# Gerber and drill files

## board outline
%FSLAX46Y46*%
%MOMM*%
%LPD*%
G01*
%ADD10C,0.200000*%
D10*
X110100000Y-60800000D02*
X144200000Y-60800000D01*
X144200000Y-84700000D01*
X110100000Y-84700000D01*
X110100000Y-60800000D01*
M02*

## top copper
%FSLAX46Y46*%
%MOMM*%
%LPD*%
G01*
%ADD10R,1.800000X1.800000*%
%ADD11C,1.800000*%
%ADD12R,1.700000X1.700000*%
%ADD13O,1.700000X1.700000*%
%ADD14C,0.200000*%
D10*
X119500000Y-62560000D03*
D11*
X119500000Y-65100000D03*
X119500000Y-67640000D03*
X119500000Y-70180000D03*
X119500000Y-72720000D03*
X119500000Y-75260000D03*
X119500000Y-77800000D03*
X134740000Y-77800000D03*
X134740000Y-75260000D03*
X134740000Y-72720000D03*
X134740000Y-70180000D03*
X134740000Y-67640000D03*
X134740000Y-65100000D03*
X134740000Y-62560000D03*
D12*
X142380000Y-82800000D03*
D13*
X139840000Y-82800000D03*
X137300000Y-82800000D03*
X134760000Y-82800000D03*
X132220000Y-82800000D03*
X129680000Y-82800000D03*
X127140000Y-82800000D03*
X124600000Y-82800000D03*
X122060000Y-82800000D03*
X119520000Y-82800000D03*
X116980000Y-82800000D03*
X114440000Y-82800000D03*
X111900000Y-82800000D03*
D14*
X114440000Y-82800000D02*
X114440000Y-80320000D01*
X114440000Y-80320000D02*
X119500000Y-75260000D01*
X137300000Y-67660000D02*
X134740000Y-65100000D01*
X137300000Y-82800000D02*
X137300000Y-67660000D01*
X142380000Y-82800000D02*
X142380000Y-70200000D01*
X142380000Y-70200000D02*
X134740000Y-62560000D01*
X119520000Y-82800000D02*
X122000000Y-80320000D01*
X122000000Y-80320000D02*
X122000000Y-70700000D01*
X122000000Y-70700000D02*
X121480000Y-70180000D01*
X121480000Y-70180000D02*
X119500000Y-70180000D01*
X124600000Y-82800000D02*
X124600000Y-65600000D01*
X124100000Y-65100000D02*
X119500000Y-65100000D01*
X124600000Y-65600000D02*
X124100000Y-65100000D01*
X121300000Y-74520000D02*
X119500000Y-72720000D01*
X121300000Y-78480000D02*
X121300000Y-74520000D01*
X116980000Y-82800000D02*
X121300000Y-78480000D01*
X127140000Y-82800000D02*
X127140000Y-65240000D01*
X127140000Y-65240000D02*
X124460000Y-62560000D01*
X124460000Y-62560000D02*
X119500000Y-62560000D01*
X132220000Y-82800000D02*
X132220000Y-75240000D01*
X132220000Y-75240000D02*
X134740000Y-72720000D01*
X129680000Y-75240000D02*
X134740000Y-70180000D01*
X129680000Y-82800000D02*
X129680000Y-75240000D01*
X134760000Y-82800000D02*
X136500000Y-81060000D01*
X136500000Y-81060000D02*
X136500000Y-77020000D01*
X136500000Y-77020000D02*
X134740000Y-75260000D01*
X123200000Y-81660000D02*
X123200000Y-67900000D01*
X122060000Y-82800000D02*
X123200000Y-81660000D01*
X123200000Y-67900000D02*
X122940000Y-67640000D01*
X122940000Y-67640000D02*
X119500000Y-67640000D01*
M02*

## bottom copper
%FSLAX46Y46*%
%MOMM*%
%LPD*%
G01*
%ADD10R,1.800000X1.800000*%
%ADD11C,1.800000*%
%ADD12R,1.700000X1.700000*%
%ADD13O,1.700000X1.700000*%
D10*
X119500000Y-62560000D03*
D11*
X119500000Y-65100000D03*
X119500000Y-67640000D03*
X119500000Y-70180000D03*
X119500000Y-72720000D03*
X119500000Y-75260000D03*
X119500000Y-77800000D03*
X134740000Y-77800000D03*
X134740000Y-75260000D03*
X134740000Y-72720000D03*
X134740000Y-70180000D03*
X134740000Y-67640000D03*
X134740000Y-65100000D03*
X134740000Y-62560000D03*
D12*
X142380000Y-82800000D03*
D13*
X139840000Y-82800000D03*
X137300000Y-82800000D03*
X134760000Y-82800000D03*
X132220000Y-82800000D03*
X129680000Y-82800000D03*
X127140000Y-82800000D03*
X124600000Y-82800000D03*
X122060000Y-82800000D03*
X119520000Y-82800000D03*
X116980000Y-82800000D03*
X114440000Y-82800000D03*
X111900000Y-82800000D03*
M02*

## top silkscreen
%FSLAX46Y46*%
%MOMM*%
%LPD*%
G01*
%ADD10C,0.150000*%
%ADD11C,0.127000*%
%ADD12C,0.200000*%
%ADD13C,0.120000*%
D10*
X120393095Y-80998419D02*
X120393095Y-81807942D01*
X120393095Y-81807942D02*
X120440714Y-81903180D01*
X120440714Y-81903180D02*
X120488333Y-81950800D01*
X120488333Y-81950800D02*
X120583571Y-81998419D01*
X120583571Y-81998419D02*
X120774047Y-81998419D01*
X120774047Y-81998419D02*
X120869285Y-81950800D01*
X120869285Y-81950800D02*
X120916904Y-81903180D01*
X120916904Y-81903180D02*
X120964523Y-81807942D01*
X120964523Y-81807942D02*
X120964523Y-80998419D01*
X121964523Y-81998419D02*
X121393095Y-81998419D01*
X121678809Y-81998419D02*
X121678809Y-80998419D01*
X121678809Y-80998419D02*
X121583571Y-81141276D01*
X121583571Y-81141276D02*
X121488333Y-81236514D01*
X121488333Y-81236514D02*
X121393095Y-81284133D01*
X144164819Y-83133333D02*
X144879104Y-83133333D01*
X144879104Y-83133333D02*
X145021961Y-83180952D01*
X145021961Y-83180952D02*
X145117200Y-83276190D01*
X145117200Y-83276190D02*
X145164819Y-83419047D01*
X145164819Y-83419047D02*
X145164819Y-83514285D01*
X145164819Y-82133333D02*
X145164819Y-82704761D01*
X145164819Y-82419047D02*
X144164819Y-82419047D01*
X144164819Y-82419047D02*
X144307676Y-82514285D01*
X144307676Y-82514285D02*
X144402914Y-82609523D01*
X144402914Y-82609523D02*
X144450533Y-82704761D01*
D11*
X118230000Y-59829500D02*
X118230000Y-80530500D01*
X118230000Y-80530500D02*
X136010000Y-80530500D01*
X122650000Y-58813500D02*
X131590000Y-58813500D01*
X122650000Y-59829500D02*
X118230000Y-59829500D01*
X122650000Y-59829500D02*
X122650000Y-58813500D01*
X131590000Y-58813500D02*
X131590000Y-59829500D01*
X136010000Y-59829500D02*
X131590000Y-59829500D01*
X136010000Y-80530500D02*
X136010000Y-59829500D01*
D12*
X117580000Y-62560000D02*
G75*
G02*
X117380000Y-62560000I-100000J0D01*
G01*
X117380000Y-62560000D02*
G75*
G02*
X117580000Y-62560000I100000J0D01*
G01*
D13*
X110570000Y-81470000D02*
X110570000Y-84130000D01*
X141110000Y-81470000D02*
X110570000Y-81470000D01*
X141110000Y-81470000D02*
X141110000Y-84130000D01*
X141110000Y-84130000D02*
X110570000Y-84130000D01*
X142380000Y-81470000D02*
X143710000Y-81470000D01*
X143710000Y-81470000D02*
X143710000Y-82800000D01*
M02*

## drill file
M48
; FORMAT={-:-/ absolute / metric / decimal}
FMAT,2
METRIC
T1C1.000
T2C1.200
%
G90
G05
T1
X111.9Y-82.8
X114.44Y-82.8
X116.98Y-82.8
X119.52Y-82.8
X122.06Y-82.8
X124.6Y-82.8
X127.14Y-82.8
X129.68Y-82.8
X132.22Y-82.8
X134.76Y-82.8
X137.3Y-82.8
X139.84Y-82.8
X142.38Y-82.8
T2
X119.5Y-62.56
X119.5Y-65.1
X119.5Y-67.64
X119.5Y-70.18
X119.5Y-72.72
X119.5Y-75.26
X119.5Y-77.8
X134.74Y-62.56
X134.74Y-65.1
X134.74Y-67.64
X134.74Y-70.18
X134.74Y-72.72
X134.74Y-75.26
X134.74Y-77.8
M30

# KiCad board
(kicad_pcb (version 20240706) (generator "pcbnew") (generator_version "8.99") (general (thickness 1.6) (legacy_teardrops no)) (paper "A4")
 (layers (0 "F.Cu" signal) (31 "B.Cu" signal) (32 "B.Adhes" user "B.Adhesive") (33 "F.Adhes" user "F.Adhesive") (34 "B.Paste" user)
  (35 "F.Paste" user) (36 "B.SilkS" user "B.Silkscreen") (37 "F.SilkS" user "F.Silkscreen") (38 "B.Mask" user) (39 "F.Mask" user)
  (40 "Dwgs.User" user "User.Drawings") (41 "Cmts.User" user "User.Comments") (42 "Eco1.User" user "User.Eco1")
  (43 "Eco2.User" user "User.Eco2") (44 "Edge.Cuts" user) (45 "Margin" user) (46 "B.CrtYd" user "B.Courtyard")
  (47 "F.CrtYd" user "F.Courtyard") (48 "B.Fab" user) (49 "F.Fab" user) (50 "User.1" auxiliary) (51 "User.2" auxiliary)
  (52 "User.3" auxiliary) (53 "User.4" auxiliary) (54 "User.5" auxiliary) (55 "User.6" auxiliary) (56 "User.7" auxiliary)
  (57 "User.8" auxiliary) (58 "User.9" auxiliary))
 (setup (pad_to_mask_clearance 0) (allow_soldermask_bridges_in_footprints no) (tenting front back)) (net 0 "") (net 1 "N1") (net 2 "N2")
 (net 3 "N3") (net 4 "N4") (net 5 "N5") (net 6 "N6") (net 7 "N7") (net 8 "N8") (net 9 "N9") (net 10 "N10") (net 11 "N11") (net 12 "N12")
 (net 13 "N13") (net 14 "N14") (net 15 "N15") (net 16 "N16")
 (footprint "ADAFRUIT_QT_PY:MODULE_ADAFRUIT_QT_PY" (layer "F.Cu") (at 127.12 70.18)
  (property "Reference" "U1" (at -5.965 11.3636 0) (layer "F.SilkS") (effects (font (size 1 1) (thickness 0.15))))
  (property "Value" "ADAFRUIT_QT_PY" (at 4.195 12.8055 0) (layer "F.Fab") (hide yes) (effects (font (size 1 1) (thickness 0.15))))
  (fp_line (start -8.89 -10.3505) (end -8.89 10.3505) (stroke (width 0.127) (type solid)) (layer "F.SilkS"))
  (fp_line (start -8.89 10.3505) (end 8.89 10.3505) (stroke (width 0.127) (type solid)) (layer "F.SilkS"))
  (fp_line (start -4.47 -11.3665) (end 4.47 -11.3665) (stroke (width 0.127) (type solid)) (layer "F.SilkS"))
  (fp_line (start -4.47 -10.3505) (end -8.89 -10.3505) (stroke (width 0.127) (type solid)) (layer "F.SilkS"))
  (fp_line (start -4.47 -10.3505) (end -4.47 -11.3665) (stroke (width 0.127) (type solid)) (layer "F.SilkS"))
  (fp_line (start 4.47 -11.3665) (end 4.47 -10.3505) (stroke (width 0.127) (type solid)) (layer "F.SilkS"))
  (fp_line (start 8.89 -10.3505) (end 4.47 -10.3505) (stroke (width 0.127) (type solid)) (layer "F.SilkS"))
  (fp_line (start 8.89 10.3505) (end 8.89 -10.3505) (stroke (width 0.127) (type solid)) (layer "F.SilkS"))
  (fp_circle (center -9.64 -7.62) (end -9.54 -7.62) (stroke (width 0.2) (type solid)) (fill none) (layer "F.SilkS"))
  (pad "1" thru_hole rect (at -7.62 -7.62) (size 1.8 1.8) (drill 1.2) (layers "*.Cu" "*.Mask") (remove_unused_layers no) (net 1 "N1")
   (solder_mask_margin 0.102))
  (pad "2" thru_hole circle (at -7.62 -5.08) (size 1.8 1.8) (drill 1.2) (layers "*.Cu" "*.Mask") (remove_unused_layers no) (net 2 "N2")
   (solder_mask_margin 0.102))
  (pad "3" thru_hole circle (at -7.62 -2.54) (size 1.8 1.8) (drill 1.2) (layers "*.Cu" "*.Mask") (remove_unused_layers no) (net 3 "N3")
   (solder_mask_margin 0.102))
  (pad "4" thru_hole circle (at -7.62 0) (size 1.8 1.8) (drill 1.2) (layers "*.Cu" "*.Mask") (remove_unused_layers no) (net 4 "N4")
   (solder_mask_margin 0.102))
  (pad "5" thru_hole circle (at -7.62 2.54) (size 1.8 1.8) (drill 1.2) (layers "*.Cu" "*.Mask") (remove_unused_layers no) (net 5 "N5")
   (solder_mask_margin 0.102))
  (pad "6" thru_hole circle (at -7.62 5.08) (size 1.8 1.8) (drill 1.2) (layers "*.Cu" "*.Mask") (remove_unused_layers no) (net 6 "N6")
   (solder_mask_margin 0.102))
  (pad "7" thru_hole circle (at -7.62 7.62) (size 1.8 1.8) (drill 1.2) (layers "*.Cu" "*.Mask") (remove_unused_layers no) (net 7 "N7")
   (solder_mask_margin 0.102))
  (pad "8" thru_hole circle (at 7.62 7.62) (size 1.8 1.8) (drill 1.2) (layers "*.Cu" "*.Mask") (remove_unused_layers no) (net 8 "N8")
   (solder_mask_margin 0.102))
  (pad "9" thru_hole circle (at 7.62 5.08) (size 1.8 1.8) (drill 1.2) (layers "*.Cu" "*.Mask") (remove_unused_layers no) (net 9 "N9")
   (solder_mask_margin 0.102))
  (pad "10" thru_hole circle (at 7.62 2.54) (size 1.8 1.8) (drill 1.2) (layers "*.Cu" "*.Mask") (remove_unused_layers no) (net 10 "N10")
   (solder_mask_margin 0.102))
  (pad "11" thru_hole circle (at 7.62 0) (size 1.8 1.8) (drill 1.2) (layers "*.Cu" "*.Mask") (remove_unused_layers no) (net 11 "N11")
   (solder_mask_margin 0.102))
  (pad "12" thru_hole circle (at 7.62 -2.54) (size 1.8 1.8) (drill 1.2) (layers "*.Cu" "*.Mask") (remove_unused_layers no) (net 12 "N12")
   (solder_mask_margin 0.102))
  (pad "13" thru_hole circle (at 7.62 -5.08) (size 1.8 1.8) (drill 1.2) (layers "*.Cu" "*.Mask") (remove_unused_layers no) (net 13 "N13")
   (solder_mask_margin 0.102))
  (pad "14" thru_hole circle (at 7.62 -7.62) (size 1.8 1.8) (drill 1.2) (layers "*.Cu" "*.Mask") (remove_unused_layers no) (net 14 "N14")
   (solder_mask_margin 0.102)))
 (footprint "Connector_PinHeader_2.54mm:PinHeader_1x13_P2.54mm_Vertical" (layer "F.Cu") (at 142.38 82.8 -90)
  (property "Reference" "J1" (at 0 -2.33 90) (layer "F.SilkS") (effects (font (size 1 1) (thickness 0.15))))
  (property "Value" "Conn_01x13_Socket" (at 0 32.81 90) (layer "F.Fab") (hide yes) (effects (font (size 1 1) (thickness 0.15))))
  (fp_line (start -1.33 31.81) (end 1.33 31.81) (stroke (width 0.12) (type solid)) (layer "F.SilkS"))
  (fp_line (start -1.33 1.27) (end -1.33 31.81) (stroke (width 0.12) (type solid)) (layer "F.SilkS"))
  (fp_line (start -1.33 1.27) (end 1.33 1.27) (stroke (width 0.12) (type solid)) (layer "F.SilkS"))
  (fp_line (start 1.33 1.27) (end 1.33 31.81) (stroke (width 0.12) (type solid)) (layer "F.SilkS"))
  (fp_line (start -1.33 0) (end -1.33 -1.33) (stroke (width 0.12) (type solid)) (layer "F.SilkS"))
  (fp_line (start -1.33 -1.33) (end 0 -1.33) (stroke (width 0.12) (type solid)) (layer "F.SilkS"))
  (pad "1" thru_hole rect (at 0 0 270) (size 1.7 1.7) (drill 1) (layers "*.Cu" "*.Mask") (remove_unused_layers no) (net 14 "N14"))
  (pad "2" thru_hole oval (at 0 2.54 270) (size 1.7 1.7) (drill 1) (layers "*.Cu" "*.Mask") (remove_unused_layers no) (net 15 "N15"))
  (pad "3" thru_hole oval (at 0 5.08 270) (size 1.7 1.7) (drill 1) (layers "*.Cu" "*.Mask") (remove_unused_layers no) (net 13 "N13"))
  (pad "4" thru_hole oval (at 0 7.62 270) (size 1.7 1.7) (drill 1) (layers "*.Cu" "*.Mask") (remove_unused_layers no) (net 9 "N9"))
  (pad "5" thru_hole oval (at 0 10.16 270) (size 1.7 1.7) (drill 1) (layers "*.Cu" "*.Mask") (remove_unused_layers no) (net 10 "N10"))
  (pad "6" thru_hole oval (at 0 12.7 270) (size 1.7 1.7) (drill 1) (layers "*.Cu" "*.Mask") (remove_unused_layers no) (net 11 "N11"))
  (pad "7" thru_hole oval (at 0 15.24 270) (size 1.7 1.7) (drill 1) (layers "*.Cu" "*.Mask") (remove_unused_layers no) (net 1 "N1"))
  (pad "8" thru_hole oval (at 0 17.78 270) (size 1.7 1.7) (drill 1) (layers "*.Cu" "*.Mask") (remove_unused_layers no) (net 2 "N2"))
  (pad "9" thru_hole oval (at 0 20.32 270) (size 1.7 1.7) (drill 1) (layers "*.Cu" "*.Mask") (remove_unused_layers no) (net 3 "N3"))
  (pad "10" thru_hole oval (at 0 22.86 270) (size 1.7 1.7) (drill 1) (layers "*.Cu" "*.Mask") (remove_unused_layers no) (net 4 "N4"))
  (pad "11" thru_hole oval (at 0 25.4 270) (size 1.7 1.7) (drill 1) (layers "*.Cu" "*.Mask") (remove_unused_layers no) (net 5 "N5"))
  (pad "12" thru_hole oval (at 0 27.94 270) (size 1.7 1.7) (drill 1) (layers "*.Cu" "*.Mask") (remove_unused_layers no) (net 6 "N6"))
  (pad "13" thru_hole oval (at 0 30.48 270) (size 1.7 1.7) (drill 1) (layers "*.Cu" "*.Mask") (remove_unused_layers no) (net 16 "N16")))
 (gr_rect (start 110.1 60.8) (end 144.2 84.7) (stroke (width 0.2) (type default)) (fill none) (layer "Edge.Cuts"))
 (segment (start 114.44 82.8) (end 114.44 80.32) (width 0.2) (layer "F.Cu") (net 6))
 (segment (start 114.44 80.32) (end 119.5 75.26) (width 0.2) (layer "F.Cu") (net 6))
 (segment (start 137.3 67.66) (end 134.74 65.1) (width 0.2) (layer "F.Cu") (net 13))
 (segment (start 137.3 82.8) (end 137.3 67.66) (width 0.2) (layer "F.Cu") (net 13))
 (segment (start 142.38 82.8) (end 142.38 70.2) (width 0.2) (layer "F.Cu") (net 14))
 (segment (start 142.38 70.2) (end 134.74 62.56) (width 0.2) (layer "F.Cu") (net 14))
 (segment (start 119.52 82.8) (end 122 80.32) (width 0.2) (layer "F.Cu") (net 4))
 (segment (start 122 80.32) (end 122 70.7) (width 0.2) (layer "F.Cu") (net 4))
 (segment (start 122 70.7) (end 121.48 70.18) (width 0.2) (layer "F.Cu") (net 4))
 (segment (start 121.48 70.18) (end 119.5 70.18) (width 0.2) (layer "F.Cu") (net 4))
 (segment (start 124.6 82.8) (end 124.6 65.6) (width 0.2) (layer "F.Cu") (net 2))
 (segment (start 124.1 65.1) (end 119.5 65.1) (width 0.2) (layer "F.Cu") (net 2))
 (segment (start 124.6 65.6) (end 124.1 65.1) (width 0.2) (layer "F.Cu") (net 2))
 (segment (start 121.3 74.52) (end 119.5 72.72) (width 0.2) (layer "F.Cu") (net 5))
 (segment (start 121.3 78.48) (end 121.3 74.52) (width 0.2) (layer "F.Cu") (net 5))
 (segment (start 116.98 82.8) (end 121.3 78.48) (width 0.2) (layer "F.Cu") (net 5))
 (segment (start 127.14 82.8) (end 127.14 65.24) (width 0.2) (layer "F.Cu") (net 1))
 (segment (start 127.14 65.24) (end 124.46 62.56) (width 0.2) (layer "F.Cu") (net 1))
 (segment (start 124.46 62.56) (end 119.5 62.56) (width 0.2) (layer "F.Cu") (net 1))
 (segment (start 132.22 82.8) (end 132.22 75.24) (width 0.2) (layer "F.Cu") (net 10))
 (segment (start 132.22 75.24) (end 134.74 72.72) (width 0.2) (layer "F.Cu") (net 10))
 (segment (start 129.68 75.24) (end 134.74 70.18) (width 0.2) (layer "F.Cu") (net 11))
 (segment (start 129.68 82.8) (end 129.68 75.24) (width 0.2) (layer "F.Cu") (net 11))
 (segment (start 134.76 82.8) (end 136.5 81.06) (width 0.2) (layer "F.Cu") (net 9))
 (segment (start 136.5 81.06) (end 136.5 77.02) (width 0.2) (layer "F.Cu") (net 9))
 (segment (start 136.5 77.02) (end 134.74 75.26) (width 0.2) (layer "F.Cu") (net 9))
 (segment (start 123.2 81.66) (end 123.2 67.9) (width 0.2) (layer "F.Cu") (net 3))
 (segment (start 122.06 82.8) (end 123.2 81.66) (width 0.2) (layer "F.Cu") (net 3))
 (segment (start 123.2 67.9) (end 122.94 67.64) (width 0.2) (layer "F.Cu") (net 3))
 (segment (start 122.94 67.64) (end 119.5 67.64) (width 0.2) (layer "F.Cu") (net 3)))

